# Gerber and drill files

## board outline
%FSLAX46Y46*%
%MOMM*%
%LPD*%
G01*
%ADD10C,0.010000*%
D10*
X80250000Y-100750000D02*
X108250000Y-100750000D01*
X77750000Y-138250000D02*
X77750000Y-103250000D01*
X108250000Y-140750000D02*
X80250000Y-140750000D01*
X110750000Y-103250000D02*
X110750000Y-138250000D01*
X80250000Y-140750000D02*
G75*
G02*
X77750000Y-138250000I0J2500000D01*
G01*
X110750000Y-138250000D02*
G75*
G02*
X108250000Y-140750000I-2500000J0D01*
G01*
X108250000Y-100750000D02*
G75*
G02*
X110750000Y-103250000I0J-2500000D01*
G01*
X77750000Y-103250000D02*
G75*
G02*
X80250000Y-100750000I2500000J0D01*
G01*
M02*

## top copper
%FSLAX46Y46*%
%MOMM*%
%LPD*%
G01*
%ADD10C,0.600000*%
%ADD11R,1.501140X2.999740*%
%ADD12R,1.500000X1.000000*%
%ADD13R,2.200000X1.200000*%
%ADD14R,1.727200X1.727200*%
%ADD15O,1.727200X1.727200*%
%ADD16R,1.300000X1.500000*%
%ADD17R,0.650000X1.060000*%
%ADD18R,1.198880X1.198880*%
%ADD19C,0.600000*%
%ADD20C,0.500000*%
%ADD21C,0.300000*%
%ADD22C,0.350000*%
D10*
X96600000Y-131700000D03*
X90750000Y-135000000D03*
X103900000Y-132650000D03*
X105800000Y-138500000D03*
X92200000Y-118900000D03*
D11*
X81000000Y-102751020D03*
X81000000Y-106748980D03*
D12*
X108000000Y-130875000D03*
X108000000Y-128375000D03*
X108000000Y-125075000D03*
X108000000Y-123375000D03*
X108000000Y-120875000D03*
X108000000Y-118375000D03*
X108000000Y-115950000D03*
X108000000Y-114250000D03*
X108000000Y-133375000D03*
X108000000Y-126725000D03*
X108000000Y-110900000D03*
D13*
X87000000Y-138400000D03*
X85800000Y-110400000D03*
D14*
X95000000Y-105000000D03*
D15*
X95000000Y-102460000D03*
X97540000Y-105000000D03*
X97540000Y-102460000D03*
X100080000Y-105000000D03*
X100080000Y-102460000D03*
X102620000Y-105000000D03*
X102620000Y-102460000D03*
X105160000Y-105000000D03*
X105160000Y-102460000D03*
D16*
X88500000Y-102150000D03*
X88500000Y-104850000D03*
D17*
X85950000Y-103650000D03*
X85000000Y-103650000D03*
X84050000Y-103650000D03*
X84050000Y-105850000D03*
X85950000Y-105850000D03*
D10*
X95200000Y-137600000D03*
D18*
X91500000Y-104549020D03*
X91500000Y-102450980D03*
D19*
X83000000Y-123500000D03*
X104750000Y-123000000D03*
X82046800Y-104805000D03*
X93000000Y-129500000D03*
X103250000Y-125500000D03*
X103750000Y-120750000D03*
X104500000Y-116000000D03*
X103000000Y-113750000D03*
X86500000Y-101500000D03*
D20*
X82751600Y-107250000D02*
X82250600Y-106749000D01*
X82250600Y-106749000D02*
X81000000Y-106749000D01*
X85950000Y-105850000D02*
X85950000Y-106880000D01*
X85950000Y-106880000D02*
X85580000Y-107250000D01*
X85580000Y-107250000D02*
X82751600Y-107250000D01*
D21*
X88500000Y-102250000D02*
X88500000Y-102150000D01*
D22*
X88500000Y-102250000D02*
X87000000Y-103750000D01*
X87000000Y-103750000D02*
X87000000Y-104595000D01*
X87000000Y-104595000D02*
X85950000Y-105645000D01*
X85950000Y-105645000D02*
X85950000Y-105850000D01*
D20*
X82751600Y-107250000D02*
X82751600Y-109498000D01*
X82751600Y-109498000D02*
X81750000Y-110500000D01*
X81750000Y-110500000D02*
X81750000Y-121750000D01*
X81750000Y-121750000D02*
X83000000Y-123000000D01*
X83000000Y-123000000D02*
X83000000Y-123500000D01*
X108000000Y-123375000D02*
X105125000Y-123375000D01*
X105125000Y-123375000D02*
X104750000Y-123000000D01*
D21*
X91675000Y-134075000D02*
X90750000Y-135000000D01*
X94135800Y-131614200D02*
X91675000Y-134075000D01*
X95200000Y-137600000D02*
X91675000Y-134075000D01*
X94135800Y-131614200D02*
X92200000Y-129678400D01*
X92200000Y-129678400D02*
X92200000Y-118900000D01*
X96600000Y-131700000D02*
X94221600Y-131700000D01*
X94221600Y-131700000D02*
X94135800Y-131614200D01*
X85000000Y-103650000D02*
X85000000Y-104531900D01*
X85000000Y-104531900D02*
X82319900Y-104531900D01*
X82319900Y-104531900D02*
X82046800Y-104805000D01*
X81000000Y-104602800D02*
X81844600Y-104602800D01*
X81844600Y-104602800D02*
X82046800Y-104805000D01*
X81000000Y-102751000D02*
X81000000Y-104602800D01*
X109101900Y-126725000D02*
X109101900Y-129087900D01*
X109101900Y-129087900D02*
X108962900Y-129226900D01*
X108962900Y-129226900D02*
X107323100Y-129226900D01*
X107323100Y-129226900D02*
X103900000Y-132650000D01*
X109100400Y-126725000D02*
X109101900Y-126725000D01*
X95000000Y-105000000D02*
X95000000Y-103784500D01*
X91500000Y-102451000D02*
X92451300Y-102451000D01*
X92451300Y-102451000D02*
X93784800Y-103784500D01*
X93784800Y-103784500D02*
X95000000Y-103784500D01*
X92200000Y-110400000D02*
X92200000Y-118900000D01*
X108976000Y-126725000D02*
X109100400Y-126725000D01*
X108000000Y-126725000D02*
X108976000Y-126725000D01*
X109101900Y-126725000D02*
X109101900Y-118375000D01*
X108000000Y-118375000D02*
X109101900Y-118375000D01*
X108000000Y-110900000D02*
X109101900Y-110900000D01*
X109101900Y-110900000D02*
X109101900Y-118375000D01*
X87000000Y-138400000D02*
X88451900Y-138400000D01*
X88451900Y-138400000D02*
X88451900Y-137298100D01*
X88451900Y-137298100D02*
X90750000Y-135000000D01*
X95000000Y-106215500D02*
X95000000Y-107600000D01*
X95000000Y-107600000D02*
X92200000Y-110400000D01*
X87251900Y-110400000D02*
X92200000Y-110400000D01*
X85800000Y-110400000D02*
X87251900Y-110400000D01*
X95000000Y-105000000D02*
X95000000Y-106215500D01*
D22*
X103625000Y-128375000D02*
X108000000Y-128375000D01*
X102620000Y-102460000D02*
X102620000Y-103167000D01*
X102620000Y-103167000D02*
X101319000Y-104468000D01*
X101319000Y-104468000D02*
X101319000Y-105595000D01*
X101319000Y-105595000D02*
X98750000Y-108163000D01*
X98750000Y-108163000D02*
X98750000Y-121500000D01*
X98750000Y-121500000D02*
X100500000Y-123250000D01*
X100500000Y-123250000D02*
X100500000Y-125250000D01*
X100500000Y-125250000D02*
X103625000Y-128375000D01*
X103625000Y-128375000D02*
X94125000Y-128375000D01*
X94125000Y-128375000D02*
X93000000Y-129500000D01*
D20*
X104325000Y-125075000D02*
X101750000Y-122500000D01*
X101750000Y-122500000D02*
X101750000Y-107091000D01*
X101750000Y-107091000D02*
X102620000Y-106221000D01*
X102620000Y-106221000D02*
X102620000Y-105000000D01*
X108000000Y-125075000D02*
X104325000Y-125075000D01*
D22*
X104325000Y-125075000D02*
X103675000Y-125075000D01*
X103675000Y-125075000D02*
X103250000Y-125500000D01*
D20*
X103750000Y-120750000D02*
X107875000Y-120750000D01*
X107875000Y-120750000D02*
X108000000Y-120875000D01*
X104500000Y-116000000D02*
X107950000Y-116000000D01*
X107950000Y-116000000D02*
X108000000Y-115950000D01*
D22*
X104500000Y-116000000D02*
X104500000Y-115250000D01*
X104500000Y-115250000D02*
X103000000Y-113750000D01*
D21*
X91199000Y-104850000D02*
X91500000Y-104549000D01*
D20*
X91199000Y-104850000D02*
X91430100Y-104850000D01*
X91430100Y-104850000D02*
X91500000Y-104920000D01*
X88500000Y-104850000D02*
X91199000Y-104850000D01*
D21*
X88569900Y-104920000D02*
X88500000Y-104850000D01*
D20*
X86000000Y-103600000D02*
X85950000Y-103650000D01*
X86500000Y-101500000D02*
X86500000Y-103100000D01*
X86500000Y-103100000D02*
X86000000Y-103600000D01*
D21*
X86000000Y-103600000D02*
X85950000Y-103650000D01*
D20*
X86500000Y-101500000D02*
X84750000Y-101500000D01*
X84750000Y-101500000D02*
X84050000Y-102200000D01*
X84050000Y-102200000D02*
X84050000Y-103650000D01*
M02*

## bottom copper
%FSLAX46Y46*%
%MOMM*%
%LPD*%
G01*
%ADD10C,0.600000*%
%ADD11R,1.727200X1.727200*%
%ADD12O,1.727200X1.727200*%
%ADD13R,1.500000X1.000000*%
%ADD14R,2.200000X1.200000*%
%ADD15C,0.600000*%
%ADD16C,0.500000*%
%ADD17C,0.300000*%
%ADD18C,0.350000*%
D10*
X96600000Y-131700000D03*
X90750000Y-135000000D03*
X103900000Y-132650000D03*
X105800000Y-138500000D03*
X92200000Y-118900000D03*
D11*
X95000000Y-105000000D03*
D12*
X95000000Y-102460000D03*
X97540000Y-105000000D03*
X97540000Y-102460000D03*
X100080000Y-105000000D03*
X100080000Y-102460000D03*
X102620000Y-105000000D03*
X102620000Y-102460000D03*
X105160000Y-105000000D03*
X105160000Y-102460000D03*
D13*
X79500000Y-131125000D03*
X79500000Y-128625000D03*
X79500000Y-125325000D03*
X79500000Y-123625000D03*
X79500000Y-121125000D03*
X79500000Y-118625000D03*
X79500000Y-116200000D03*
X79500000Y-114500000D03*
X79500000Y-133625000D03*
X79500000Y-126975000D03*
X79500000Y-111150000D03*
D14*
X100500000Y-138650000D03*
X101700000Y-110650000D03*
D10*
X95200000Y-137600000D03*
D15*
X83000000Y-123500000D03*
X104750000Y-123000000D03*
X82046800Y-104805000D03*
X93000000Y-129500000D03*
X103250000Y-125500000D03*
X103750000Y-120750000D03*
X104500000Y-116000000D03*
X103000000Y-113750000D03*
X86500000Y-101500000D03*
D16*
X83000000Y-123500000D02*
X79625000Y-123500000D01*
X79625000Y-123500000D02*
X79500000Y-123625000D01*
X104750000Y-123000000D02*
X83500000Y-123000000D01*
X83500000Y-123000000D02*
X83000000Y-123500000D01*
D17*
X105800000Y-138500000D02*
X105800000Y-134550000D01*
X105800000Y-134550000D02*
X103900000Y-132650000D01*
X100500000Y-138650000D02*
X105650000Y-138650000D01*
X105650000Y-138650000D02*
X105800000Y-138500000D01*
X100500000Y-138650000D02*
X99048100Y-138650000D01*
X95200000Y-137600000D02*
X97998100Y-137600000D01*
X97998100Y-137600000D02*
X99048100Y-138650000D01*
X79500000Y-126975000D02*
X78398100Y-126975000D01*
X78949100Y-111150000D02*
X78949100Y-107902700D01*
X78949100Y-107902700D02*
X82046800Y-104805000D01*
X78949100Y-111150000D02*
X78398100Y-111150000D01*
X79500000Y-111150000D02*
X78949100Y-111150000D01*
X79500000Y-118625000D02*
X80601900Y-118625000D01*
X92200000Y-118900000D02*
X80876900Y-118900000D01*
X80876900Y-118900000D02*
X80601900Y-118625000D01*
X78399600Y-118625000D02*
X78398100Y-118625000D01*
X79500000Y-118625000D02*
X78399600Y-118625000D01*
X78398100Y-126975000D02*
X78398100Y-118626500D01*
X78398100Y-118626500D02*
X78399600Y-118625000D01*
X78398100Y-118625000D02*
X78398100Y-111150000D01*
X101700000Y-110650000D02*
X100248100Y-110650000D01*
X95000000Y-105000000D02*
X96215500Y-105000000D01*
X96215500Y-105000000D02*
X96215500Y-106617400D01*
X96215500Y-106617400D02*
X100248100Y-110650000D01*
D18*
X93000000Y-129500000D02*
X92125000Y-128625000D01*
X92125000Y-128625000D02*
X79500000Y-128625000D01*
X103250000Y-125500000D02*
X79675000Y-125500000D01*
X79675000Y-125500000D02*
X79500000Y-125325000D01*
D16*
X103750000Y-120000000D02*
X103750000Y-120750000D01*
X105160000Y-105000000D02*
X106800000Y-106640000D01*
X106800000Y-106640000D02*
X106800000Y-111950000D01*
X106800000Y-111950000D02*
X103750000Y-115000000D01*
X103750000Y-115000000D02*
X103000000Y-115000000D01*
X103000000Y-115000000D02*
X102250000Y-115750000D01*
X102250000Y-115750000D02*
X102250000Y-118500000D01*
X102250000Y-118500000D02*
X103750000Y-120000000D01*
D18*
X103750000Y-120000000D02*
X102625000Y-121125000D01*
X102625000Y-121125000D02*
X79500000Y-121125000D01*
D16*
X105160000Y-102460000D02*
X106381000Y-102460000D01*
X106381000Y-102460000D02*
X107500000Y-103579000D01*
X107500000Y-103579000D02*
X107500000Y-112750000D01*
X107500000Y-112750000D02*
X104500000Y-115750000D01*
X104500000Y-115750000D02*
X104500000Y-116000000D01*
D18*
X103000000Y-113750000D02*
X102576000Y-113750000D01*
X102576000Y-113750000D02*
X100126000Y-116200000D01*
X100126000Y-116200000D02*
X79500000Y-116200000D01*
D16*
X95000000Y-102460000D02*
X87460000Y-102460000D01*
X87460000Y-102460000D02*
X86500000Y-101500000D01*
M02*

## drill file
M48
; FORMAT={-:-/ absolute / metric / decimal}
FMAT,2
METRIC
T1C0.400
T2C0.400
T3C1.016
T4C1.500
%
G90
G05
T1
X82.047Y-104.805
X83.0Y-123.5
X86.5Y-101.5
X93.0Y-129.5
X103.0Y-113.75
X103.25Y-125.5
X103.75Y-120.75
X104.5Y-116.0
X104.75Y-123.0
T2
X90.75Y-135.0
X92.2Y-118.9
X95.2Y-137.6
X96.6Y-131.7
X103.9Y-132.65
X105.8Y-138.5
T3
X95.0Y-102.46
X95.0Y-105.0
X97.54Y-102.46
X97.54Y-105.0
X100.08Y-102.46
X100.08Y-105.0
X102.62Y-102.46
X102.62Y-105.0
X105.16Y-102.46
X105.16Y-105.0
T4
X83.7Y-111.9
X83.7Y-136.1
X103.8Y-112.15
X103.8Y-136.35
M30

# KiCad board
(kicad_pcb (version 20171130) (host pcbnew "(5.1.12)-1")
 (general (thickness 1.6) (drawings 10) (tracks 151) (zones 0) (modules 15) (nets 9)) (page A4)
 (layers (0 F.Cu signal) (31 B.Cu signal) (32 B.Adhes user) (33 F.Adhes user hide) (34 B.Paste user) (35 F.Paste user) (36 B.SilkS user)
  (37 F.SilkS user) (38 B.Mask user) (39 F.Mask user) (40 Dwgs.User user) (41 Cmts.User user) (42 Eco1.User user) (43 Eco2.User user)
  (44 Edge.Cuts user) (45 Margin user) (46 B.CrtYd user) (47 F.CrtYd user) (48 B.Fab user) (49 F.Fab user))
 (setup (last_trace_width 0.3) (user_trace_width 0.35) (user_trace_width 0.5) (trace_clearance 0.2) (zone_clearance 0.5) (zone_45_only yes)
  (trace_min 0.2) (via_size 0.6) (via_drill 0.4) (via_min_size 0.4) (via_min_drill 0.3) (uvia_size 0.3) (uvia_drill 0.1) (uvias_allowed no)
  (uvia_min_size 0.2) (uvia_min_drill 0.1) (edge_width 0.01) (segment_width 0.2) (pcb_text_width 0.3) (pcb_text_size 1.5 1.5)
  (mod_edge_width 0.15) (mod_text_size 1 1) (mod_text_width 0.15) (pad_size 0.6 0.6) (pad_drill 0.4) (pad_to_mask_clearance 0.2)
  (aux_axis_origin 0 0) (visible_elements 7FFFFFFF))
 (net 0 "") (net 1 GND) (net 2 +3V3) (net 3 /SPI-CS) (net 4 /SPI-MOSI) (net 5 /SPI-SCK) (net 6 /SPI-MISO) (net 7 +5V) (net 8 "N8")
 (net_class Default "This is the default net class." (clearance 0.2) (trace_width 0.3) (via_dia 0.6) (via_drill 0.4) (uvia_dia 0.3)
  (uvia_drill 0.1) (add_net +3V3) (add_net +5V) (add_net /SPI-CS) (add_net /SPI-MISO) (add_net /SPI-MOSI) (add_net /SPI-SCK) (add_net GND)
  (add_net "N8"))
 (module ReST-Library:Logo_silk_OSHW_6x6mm (layer B.Cu) (at 86.868 123.444 270)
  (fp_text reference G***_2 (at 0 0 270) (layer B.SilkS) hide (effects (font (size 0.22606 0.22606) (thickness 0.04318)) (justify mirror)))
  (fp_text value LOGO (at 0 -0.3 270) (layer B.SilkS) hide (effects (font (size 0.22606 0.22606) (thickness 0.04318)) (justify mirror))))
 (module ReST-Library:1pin (layer F.Cu) (at 96.6 131.7) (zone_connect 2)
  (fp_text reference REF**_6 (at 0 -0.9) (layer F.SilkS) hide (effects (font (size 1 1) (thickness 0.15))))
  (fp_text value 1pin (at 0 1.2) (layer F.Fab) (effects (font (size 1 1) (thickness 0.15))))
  (pad GND thru_hole circle (at 0 0) (size 0.6 0.6) (drill 0.4) (layers *.Cu *.Mask F.SilkS) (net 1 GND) (zone_connect 2)))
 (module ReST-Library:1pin (layer F.Cu) (at 90.75 135) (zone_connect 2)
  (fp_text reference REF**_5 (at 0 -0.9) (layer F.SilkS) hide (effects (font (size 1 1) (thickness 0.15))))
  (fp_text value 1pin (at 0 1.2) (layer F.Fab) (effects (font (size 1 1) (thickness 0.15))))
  (pad GND thru_hole circle (at 0 0) (size 0.6 0.6) (drill 0.4) (layers *.Cu *.Mask F.SilkS) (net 1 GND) (zone_connect 2)))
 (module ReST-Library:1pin (layer F.Cu) (at 103.9 132.65) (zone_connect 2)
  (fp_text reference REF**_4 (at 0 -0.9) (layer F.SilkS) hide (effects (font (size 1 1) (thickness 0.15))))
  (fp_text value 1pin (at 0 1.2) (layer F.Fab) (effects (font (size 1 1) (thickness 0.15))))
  (pad GND thru_hole circle (at 0 0) (size 0.6 0.6) (drill 0.4) (layers *.Cu *.Mask F.SilkS) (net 1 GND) (zone_connect 2)))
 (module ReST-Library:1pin (layer F.Cu) (at 105.8 138.5) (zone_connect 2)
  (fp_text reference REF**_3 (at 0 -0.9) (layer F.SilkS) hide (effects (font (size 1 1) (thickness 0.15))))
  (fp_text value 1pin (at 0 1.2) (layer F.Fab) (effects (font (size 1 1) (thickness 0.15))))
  (pad GND thru_hole circle (at 0 0) (size 0.6 0.6) (drill 0.4) (layers *.Cu *.Mask F.SilkS) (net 1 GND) (zone_connect 2)))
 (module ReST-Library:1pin (layer F.Cu) (at 92.2 118.9) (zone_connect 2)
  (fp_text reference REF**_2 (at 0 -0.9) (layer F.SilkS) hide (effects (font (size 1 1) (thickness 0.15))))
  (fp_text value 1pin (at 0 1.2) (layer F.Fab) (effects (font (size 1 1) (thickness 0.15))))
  (pad GND thru_hole circle (at 0 0) (size 0.6 0.6) (drill 0.4) (layers *.Cu *.Mask F.SilkS) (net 1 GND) (zone_connect 2)))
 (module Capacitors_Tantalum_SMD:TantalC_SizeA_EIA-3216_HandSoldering (layer F.Cu) (at 81 104.75 90)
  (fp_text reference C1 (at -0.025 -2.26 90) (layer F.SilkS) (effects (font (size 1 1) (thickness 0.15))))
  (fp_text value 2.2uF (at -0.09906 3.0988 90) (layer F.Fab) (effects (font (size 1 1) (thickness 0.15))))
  (pad 2 smd rect (at 1.99898 0 90) (size 2.99974 1.50114) (layers F.Cu F.Paste F.Mask) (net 1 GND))
  (pad 1 smd rect (at -1.99898 0 90) (size 2.99974 1.50114) (layers F.Cu F.Paste F.Mask) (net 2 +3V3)))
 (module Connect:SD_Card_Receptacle (layer F.Cu) (at 108 124 270) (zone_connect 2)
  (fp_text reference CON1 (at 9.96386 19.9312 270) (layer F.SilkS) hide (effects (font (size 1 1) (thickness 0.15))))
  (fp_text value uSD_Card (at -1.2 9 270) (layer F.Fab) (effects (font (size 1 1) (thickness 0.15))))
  (pad 1 smd rect (at 6.875 0 270) (size 1 1.5) (layers F.Cu F.Paste F.Mask) (zone_connect 2))
  (pad 2 smd rect (at 4.375 0 270) (size 1 1.5) (layers F.Cu F.Paste F.Mask) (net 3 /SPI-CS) (zone_connect 2))
  (pad 3 smd rect (at 1.075 0 270) (size 1 1.5) (layers F.Cu F.Paste F.Mask) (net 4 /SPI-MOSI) (zone_connect 2))
  (pad 4 smd rect (at -0.625 0 270) (size 1 1.5) (layers F.Cu F.Paste F.Mask) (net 2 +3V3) (zone_connect 2))
  (pad 5 smd rect (at -3.125 0 270) (size 1 1.5) (layers F.Cu F.Paste F.Mask) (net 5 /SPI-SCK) (zone_connect 2))
  (pad 6 smd rect (at -5.625 0 270) (size 1 1.5) (layers F.Cu F.Paste F.Mask) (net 1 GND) (zone_connect 2))
  (pad 7 smd rect (at -8.05 0 270) (size 1 1.5) (layers F.Cu F.Paste F.Mask) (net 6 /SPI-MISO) (zone_connect 2))
  (pad 8 smd rect (at -9.75 0 270) (size 1 1.5) (layers F.Cu F.Paste F.Mask) (zone_connect 2))
  (pad 9 smd rect (at 9.375 0 270) (size 1 1.5) (layers F.Cu F.Paste F.Mask) (zone_connect 2))
  (pad 10 smd rect (at 2.725 0 270) (size 1 1.5) (layers F.Cu F.Paste F.Mask) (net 1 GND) (zone_connect 2))
  (pad 11 smd rect (at -13.1 0 270) (size 1 1.5) (layers F.Cu F.Paste F.Mask) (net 1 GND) (zone_connect 2))
  (pad 12 smd rect (at 14.4 21 270) (size 1.2 2.2) (layers F.Cu F.Paste F.Mask) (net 1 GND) (zone_connect 2))
  (pad 13 smd rect (at -13.6 22.2 270) (size 1.2 2.2) (layers F.Cu F.Paste F.Mask) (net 1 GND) (zone_connect 2))
  (pad "" np_thru_hole circle (at 12.1 24.3 270) (size 1.5 1.5) (drill 1.5) (layers *.Cu *.Mask F.SilkS) (zone_connect 2))
  (pad "" np_thru_hole circle (at -12.1 24.3 270) (size 1.5 1.5) (drill 1.5) (layers *.Cu *.Mask F.SilkS) (zone_connect 2)))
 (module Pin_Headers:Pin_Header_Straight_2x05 (layer F.Cu) (at 95 105 90)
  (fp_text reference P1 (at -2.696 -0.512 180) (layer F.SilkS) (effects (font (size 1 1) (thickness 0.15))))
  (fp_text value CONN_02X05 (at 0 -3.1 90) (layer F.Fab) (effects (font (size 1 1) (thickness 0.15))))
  (pad 1 thru_hole rect (at 0 0 90) (size 1.7272 1.7272) (drill 1.016) (layers *.Cu *.Mask F.SilkS) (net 1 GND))
  (pad 2 thru_hole oval (at 2.54 0 90) (size 1.7272 1.7272) (drill 1.016) (layers *.Cu *.Mask F.SilkS) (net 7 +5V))
  (pad 3 thru_hole oval (at 0 2.54 90) (size 1.7272 1.7272) (drill 1.016) (layers *.Cu *.Mask F.SilkS))
  (pad 4 thru_hole oval (at 2.54 2.54 90) (size 1.7272 1.7272) (drill 1.016) (layers *.Cu *.Mask F.SilkS))
  (pad 5 thru_hole oval (at 0 5.08 90) (size 1.7272 1.7272) (drill 1.016) (layers *.Cu *.Mask F.SilkS))
  (pad 6 thru_hole oval (at 2.54 5.08 90) (size 1.7272 1.7272) (drill 1.016) (layers *.Cu *.Mask F.SilkS))
  (pad 7 thru_hole oval (at 0 7.62 90) (size 1.7272 1.7272) (drill 1.016) (layers *.Cu *.Mask F.SilkS) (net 4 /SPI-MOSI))
  (pad 8 thru_hole oval (at 2.54 7.62 90) (size 1.7272 1.7272) (drill 1.016) (layers *.Cu *.Mask F.SilkS) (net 3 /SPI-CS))
  (pad 9 thru_hole oval (at 0 10.16 90) (size 1.7272 1.7272) (drill 1.016) (layers *.Cu *.Mask F.SilkS) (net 5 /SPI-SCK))
  (pad 10 thru_hole oval (at 2.54 10.16 90) (size 1.7272 1.7272) (drill 1.016) (layers *.Cu *.Mask F.SilkS) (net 6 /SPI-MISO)))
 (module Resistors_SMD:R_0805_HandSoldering (layer F.Cu) (at 88.5 103.5 270)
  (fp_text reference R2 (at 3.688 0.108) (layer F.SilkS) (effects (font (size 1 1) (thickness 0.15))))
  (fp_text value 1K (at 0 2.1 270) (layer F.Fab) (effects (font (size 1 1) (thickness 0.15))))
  (pad 1 smd rect (at -1.35 0 270) (size 1.5 1.3) (layers F.Cu F.Paste F.Mask) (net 2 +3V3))
  (pad 2 smd rect (at 1.35 0 270) (size 1.5 1.3) (layers F.Cu F.Paste F.Mask) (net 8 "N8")))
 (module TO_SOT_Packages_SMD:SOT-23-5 (layer F.Cu) (at 85 104.75 270)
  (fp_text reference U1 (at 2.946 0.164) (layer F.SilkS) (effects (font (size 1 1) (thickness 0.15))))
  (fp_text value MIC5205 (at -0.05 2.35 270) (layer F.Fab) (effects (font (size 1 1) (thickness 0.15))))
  (pad 1 smd rect (at -1.1 -0.95 270) (size 1.06 0.65) (layers F.Cu F.Paste F.Mask) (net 7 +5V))
  (pad 2 smd rect (at -1.1 0 270) (size 1.06 0.65) (layers F.Cu F.Paste F.Mask) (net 1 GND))
  (pad 3 smd rect (at -1.1 0.95 270) (size 1.06 0.65) (layers F.Cu F.Paste F.Mask) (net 7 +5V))
  (pad 4 smd rect (at 1.1 0.95 270) (size 1.06 0.65) (layers F.Cu F.Paste F.Mask))
  (pad 5 smd rect (at 1.1 -0.95 270) (size 1.06 0.65) (layers F.Cu F.Paste F.Mask) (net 2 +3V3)))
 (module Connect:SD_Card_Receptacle (layer B.Cu) (at 79.5 124.25 270) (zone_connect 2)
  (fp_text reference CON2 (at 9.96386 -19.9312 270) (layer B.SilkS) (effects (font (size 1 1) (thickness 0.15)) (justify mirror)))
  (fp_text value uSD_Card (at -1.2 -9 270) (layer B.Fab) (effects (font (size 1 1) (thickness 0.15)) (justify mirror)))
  (pad 1 smd rect (at 6.875 0 270) (size 1 1.5) (layers B.Cu B.Paste B.Mask) (zone_connect 2))
  (pad 2 smd rect (at 4.375 0 270) (size 1 1.5) (layers B.Cu B.Paste B.Mask) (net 3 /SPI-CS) (zone_connect 2))
  (pad 3 smd rect (at 1.075 0 270) (size 1 1.5) (layers B.Cu B.Paste B.Mask) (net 4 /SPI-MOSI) (zone_connect 2))
  (pad 4 smd rect (at -0.625 0 270) (size 1 1.5) (layers B.Cu B.Paste B.Mask) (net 2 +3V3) (zone_connect 2))
  (pad 5 smd rect (at -3.125 0 270) (size 1 1.5) (layers B.Cu B.Paste B.Mask) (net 5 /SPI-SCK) (zone_connect 2))
  (pad 6 smd rect (at -5.625 0 270) (size 1 1.5) (layers B.Cu B.Paste B.Mask) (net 1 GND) (zone_connect 2))
  (pad 7 smd rect (at -8.05 0 270) (size 1 1.5) (layers B.Cu B.Paste B.Mask) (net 6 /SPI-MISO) (zone_connect 2))
  (pad 8 smd rect (at -9.75 0 270) (size 1 1.5) (layers B.Cu B.Paste B.Mask) (zone_connect 2))
  (pad 9 smd rect (at 9.375 0 270) (size 1 1.5) (layers B.Cu B.Paste B.Mask) (zone_connect 2))
  (pad 10 smd rect (at 2.725 0 270) (size 1 1.5) (layers B.Cu B.Paste B.Mask) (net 1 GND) (zone_connect 2))
  (pad 11 smd rect (at -13.1 0 270) (size 1 1.5) (layers B.Cu B.Paste B.Mask) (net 1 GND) (zone_connect 2))
  (pad 12 smd rect (at 14.4 -21 270) (size 1.2 2.2) (layers B.Cu B.Paste B.Mask) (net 1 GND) (zone_connect 2))
  (pad 13 smd rect (at -13.6 -22.2 270) (size 1.2 2.2) (layers B.Cu B.Paste B.Mask) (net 1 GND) (zone_connect 2))
  (pad "" np_thru_hole circle (at 12.1 -24.3 270) (size 1.5 1.5) (drill 1.5) (layers *.Cu *.Mask B.SilkS) (zone_connect 2))
  (pad "" np_thru_hole circle (at -12.1 -24.3 270) (size 1.5 1.5) (drill 1.5) (layers *.Cu *.Mask B.SilkS) (zone_connect 2)))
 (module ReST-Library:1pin (layer F.Cu) (at 95.2 137.6) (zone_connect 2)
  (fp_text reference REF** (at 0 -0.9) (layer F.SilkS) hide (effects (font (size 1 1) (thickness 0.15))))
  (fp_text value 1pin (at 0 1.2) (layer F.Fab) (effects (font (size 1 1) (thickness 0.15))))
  (pad GND thru_hole circle (at 0 0) (size 0.6 0.6) (drill 0.4) (layers *.Cu *.Mask F.SilkS) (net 1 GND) (zone_connect 2)))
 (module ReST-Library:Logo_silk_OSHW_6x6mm (layer F.Cu) (at 86.868 123.444 90)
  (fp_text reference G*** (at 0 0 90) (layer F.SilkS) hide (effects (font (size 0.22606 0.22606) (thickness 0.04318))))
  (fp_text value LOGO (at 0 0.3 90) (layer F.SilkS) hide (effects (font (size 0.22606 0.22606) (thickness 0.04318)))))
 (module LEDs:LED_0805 (layer F.Cu) (at 91.5 103.5 270)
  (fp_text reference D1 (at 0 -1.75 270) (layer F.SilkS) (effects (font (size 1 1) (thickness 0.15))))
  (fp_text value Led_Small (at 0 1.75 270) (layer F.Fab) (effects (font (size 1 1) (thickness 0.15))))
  (pad 2 smd rect (at 1.04902 0 90) (size 1.19888 1.19888) (layers F.Cu F.Paste F.Mask) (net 8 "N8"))
  (pad 1 smd rect (at -1.04902 0 90) (size 1.19888 1.19888) (layers F.Cu F.Paste F.Mask) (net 1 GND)))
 (gr_line (start 80.25 100.75) (end 108.25 100.75) (angle 90) (layer Edge.Cuts) (width 0.01))
 (gr_line (start 77.75 138.25) (end 77.75 103.25) (angle 90) (layer Edge.Cuts) (width 0.01))
 (gr_line (start 108.25 140.75) (end 80.25 140.75) (angle 90) (layer Edge.Cuts) (width 0.01))
 (gr_line (start 110.75 103.25) (end 110.75 138.25) (angle 90) (layer Edge.Cuts) (width 0.01))
 (gr_arc (start 80.25 138.25) (end 80.25 140.75) (angle 90) (layer Edge.Cuts) (width 0.01))
 (gr_arc (start 108.25 138.25) (end 110.75 138.25) (angle 90) (layer Edge.Cuts) (width 0.01))
 (gr_arc (start 108.25 103.25) (end 108.25 100.75) (angle 90) (layer Edge.Cuts) (width 0.01))
 (gr_arc (start 80.25 103.25) (end 77.75 103.25) (angle 90) (layer Edge.Cuts) (width 0.01))
 (segment (start 82.7516 107.25) (end 82.2506 106.749) (width 0.5) (layer F.Cu) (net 2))
 (segment (start 82.2506 106.749) (end 81 106.749) (width 0.5) (layer F.Cu) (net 2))
 (segment (start 85.95 105.85) (end 85.95 106.88) (width 0.5) (layer F.Cu) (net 2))
 (segment (start 85.95 106.88) (end 85.58 107.25) (width 0.5) (layer F.Cu) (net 2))
 (segment (start 85.58 107.25) (end 82.7516 107.25) (width 0.5) (layer F.Cu) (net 2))
 (segment (start 88.5 102.25) (end 88.5 102.15) (width 0.3) (layer F.Cu) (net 2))
 (segment (start 88.5 102.25) (end 87 103.75) (width 0.35) (layer F.Cu) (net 2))
 (segment (start 87 103.75) (end 87 104.595) (width 0.35) (layer F.Cu) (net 2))
 (segment (start 87 104.595) (end 85.95 105.645) (width 0.35) (layer F.Cu) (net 2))
 (segment (start 85.95 105.645) (end 85.95 105.85) (width 0.35) (layer F.Cu) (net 2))
 (segment (start 82.7516 107.25) (end 82.7516 109.498) (width 0.5) (layer F.Cu) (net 2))
 (segment (start 82.7516 109.498) (end 81.75 110.5) (width 0.5) (layer F.Cu) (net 2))
 (segment (start 81.75 110.5) (end 81.75 121.75) (width 0.5) (layer F.Cu) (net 2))
 (segment (start 81.75 121.75) (end 83 123) (width 0.5) (layer F.Cu) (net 2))
 (segment (start 83 123) (end 83 123.5) (width 0.5) (layer F.Cu) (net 2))
 (segment (start 83 123.5) (end 79.625 123.5) (width 0.5) (layer B.Cu) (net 2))
 (segment (start 79.625 123.5) (end 79.5 123.625) (width 0.5) (layer B.Cu) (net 2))
 (segment (start 108 123.375) (end 105.125 123.375) (width 0.5) (layer F.Cu) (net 2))
 (segment (start 105.125 123.375) (end 104.75 123) (width 0.5) (layer F.Cu) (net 2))
 (segment (start 104.75 123) (end 83.5 123) (width 0.5) (layer B.Cu) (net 2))
 (segment (start 83.5 123) (end 83 123.5) (width 0.5) (layer B.Cu) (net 2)) (via (at 83 123.5) (size 0.6) (layers F.Cu B.Cu) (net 2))
 (via (at 104.75 123) (size 0.6) (layers F.Cu B.Cu) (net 2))
 (segment (start 105.8 138.5) (end 105.8 134.55) (width 0.3) (layer B.Cu) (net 1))
 (segment (start 105.8 134.55) (end 103.9 132.65) (width 0.3) (layer B.Cu) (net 1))
 (segment (start 100.5 138.65) (end 105.65 138.65) (width 0.3) (layer B.Cu) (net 1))
 (segment (start 105.65 138.65) (end 105.8 138.5) (width 0.3) (layer B.Cu) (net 1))
 (segment (start 100.5 138.65) (end 99.0481 138.65) (width 0.3) (layer B.Cu) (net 1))
 (segment (start 95.2 137.6) (end 97.9981 137.6) (width 0.3) (layer B.Cu) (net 1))
 (segment (start 97.9981 137.6) (end 99.0481 138.65) (width 0.3) (layer B.Cu) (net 1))
 (segment (start 91.675 134.075) (end 90.75 135) (width 0.3) (layer F.Cu) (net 1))
 (segment (start 94.1358 131.6142) (end 91.675 134.075) (width 0.3) (layer F.Cu) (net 1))
 (segment (start 95.2 137.6) (end 91.675 134.075) (width 0.3) (layer F.Cu) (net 1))
 (segment (start 94.1358 131.6142) (end 92.2 129.6784) (width 0.3) (layer F.Cu) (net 1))
 (segment (start 92.2 129.6784) (end 92.2 118.9) (width 0.3) (layer F.Cu) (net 1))
 (segment (start 96.6 131.7) (end 94.2216 131.7) (width 0.3) (layer F.Cu) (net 1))
 (segment (start 94.2216 131.7) (end 94.1358 131.6142) (width 0.3) (layer F.Cu) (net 1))
 (segment (start 79.5 126.975) (end 78.3981 126.975) (width 0.3) (layer B.Cu) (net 1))
 (segment (start 85 103.65) (end 85 104.5319) (width 0.3) (layer F.Cu) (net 1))
 (segment (start 85 104.5319) (end 82.3199 104.5319) (width 0.3) (layer F.Cu) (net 1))
 (segment (start 82.3199 104.5319) (end 82.0468 104.805) (width 0.3) (layer F.Cu) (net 1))
 (segment (start 81 104.6028) (end 81.8446 104.6028) (width 0.3) (layer F.Cu) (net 1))
 (segment (start 81.8446 104.6028) (end 82.0468 104.805) (width 0.3) (layer F.Cu) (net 1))
 (segment (start 78.9491 111.15) (end 78.9491 107.9027) (width 0.3) (layer B.Cu) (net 1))
 (segment (start 78.9491 107.9027) (end 82.0468 104.805) (width 0.3) (layer B.Cu) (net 1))
 (segment (start 81 102.751) (end 81 104.6028) (width 0.3) (layer F.Cu) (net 1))
 (segment (start 78.9491 111.15) (end 78.3981 111.15) (width 0.3) (layer B.Cu) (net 1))
 (segment (start 79.5 111.15) (end 78.9491 111.15) (width 0.3) (layer B.Cu) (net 1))
 (segment (start 109.1019 126.725) (end 109.1019 129.0879) (width 0.3) (layer F.Cu) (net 1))
 (segment (start 109.1019 129.0879) (end 108.9629 129.2269) (width 0.3) (layer F.Cu) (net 1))
 (segment (start 108.9629 129.2269) (end 107.3231 129.2269) (width 0.3) (layer F.Cu) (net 1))
 (segment (start 107.3231 129.2269) (end 103.9 132.65) (width 0.3) (layer F.Cu) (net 1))
 (segment (start 109.1004 126.725) (end 109.1019 126.725) (width 0.3) (layer F.Cu) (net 1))
 (segment (start 95 105) (end 95 103.7845) (width 0.3) (layer F.Cu) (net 1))
 (segment (start 91.5 102.451) (end 92.4513 102.451) (width 0.3) (layer F.Cu) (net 1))
 (segment (start 92.4513 102.451) (end 93.7848 103.7845) (width 0.3) (layer F.Cu) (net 1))
 (segment (start 93.7848 103.7845) (end 95 103.7845) (width 0.3) (layer F.Cu) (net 1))
 (segment (start 79.5 118.625) (end 80.6019 118.625) (width 0.3) (layer B.Cu) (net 1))
 (segment (start 92.2 118.9) (end 80.8769 118.9) (width 0.3) (layer B.Cu) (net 1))
 (segment (start 80.8769 118.9) (end 80.6019 118.625) (width 0.3) (layer B.Cu) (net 1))
 (segment (start 78.3996 118.625) (end 78.3981 118.625) (width 0.3) (layer B.Cu) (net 1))
 (segment (start 79.5 118.625) (end 78.3996 118.625) (width 0.3) (layer B.Cu) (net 1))
 (segment (start 78.3981 126.975) (end 78.3981 118.6265) (width 0.3) (layer B.Cu) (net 1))
 (segment (start 78.3981 118.6265) (end 78.3996 118.625) (width 0.3) (layer B.Cu) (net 1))
 (segment (start 78.3981 118.625) (end 78.3981 111.15) (width 0.3) (layer B.Cu) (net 1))
 (segment (start 92.2 110.4) (end 92.2 118.9) (width 0.3) (layer F.Cu) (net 1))
 (segment (start 108.976 126.725) (end 109.1004 126.725) (width 0.3) (layer F.Cu) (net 1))
 (segment (start 108 126.725) (end 108.976 126.725) (width 0.3) (layer F.Cu) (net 1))
 (segment (start 109.1019 126.725) (end 109.1019 118.375) (width 0.3) (layer F.Cu) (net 1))
 (segment (start 108 118.375) (end 109.1019 118.375) (width 0.3) (layer F.Cu) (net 1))
 (segment (start 108 110.9) (end 109.1019 110.9) (width 0.3) (layer F.Cu) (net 1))
 (segment (start 109.1019 110.9) (end 109.1019 118.375) (width 0.3) (layer F.Cu) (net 1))
 (segment (start 87 138.4) (end 88.4519 138.4) (width 0.3) (layer F.Cu) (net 1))
 (segment (start 88.4519 138.4) (end 88.4519 137.2981) (width 0.3) (layer F.Cu) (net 1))
 (segment (start 88.4519 137.2981) (end 90.75 135) (width 0.3) (layer F.Cu) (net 1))
 (segment (start 95 106.2155) (end 95 107.6) (width 0.3) (layer F.Cu) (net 1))
 (segment (start 95 107.6) (end 92.2 110.4) (width 0.3) (layer F.Cu) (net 1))
 (segment (start 87.2519 110.4) (end 92.2 110.4) (width 0.3) (layer F.Cu) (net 1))
 (segment (start 85.8 110.4) (end 87.2519 110.4) (width 0.3) (layer F.Cu) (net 1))
 (segment (start 95 105) (end 95 106.2155) (width 0.3) (layer F.Cu) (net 1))
 (segment (start 101.7 110.65) (end 100.2481 110.65) (width 0.3) (layer B.Cu) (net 1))
 (segment (start 95 105) (end 96.2155 105) (width 0.3) (layer B.Cu) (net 1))
 (segment (start 96.2155 105) (end 96.2155 106.6174) (width 0.3) (layer B.Cu) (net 1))
 (segment (start 96.2155 106.6174) (end 100.2481 110.65) (width 0.3) (layer B.Cu) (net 1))
 (via (at 82.0468 104.805) (size 0.6) (layers F.Cu B.Cu) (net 1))
 (segment (start 103.625 128.375) (end 108 128.375) (width 0.35) (layer F.Cu) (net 3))
 (segment (start 102.62 102.46) (end 102.62 103.167) (width 0.35) (layer F.Cu) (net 3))
 (segment (start 102.62 103.167) (end 101.319 104.468) (width 0.35) (layer F.Cu) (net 3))
 (segment (start 101.319 104.468) (end 101.319 105.595) (width 0.35) (layer F.Cu) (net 3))
 (segment (start 101.319 105.595) (end 98.75 108.163) (width 0.35) (layer F.Cu) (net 3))
 (segment (start 98.75 108.163) (end 98.75 121.5) (width 0.35) (layer F.Cu) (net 3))
 (segment (start 98.75 121.5) (end 100.5 123.25) (width 0.35) (layer F.Cu) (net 3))
 (segment (start 100.5 123.25) (end 100.5 125.25) (width 0.35) (layer F.Cu) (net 3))
 (segment (start 100.5 125.25) (end 103.625 128.375) (width 0.35) (layer F.Cu) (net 3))
 (segment (start 103.625 128.375) (end 94.125 128.375) (width 0.35) (layer F.Cu) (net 3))
 (segment (start 94.125 128.375) (end 93 129.5) (width 0.35) (layer F.Cu) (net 3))
 (segment (start 93 129.5) (end 92.125 128.625) (width 0.35) (layer B.Cu) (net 3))
 (segment (start 92.125 128.625) (end 79.5 128.625) (width 0.35) (layer B.Cu) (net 3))
 (via (at 93 129.5) (size 0.6) (layers F.Cu B.Cu) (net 3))
 (segment (start 104.325 125.075) (end 101.75 122.5) (width 0.5) (layer F.Cu) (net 4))
 (segment (start 101.75 122.5) (end 101.75 107.091) (width 0.5) (layer F.Cu) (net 4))
 (segment (start 101.75 107.091) (end 102.62 106.221) (width 0.5) (layer F.Cu) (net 4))
 (segment (start 102.62 106.221) (end 102.62 105) (width 0.5) (layer F.Cu) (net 4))
 (segment (start 108 125.075) (end 104.325 125.075) (width 0.5) (layer F.Cu) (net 4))
 (segment (start 104.325 125.075) (end 103.675 125.075) (width 0.35) (layer F.Cu) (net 4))
 (segment (start 103.675 125.075) (end 103.25 125.5) (width 0.35) (layer F.Cu) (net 4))
 (segment (start 103.25 125.5) (end 79.675 125.5) (width 0.35) (layer B.Cu) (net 4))
 (segment (start 79.675 125.5) (end 79.5 125.325) (width 0.35) (layer B.Cu) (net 4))
 (via (at 103.25 125.5) (size 0.6) (layers F.Cu B.Cu) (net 4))
 (segment (start 103.75 120) (end 103.75 120.75) (width 0.5) (layer B.Cu) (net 5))
 (segment (start 105.16 105) (end 106.8 106.64) (width 0.5) (layer B.Cu) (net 5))
 (segment (start 106.8 106.64) (end 106.8 111.95) (width 0.5) (layer B.Cu) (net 5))
 (segment (start 106.8 111.95) (end 103.75 115) (width 0.5) (layer B.Cu) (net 5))
 (segment (start 103.75 115) (end 103 115) (width 0.5) (layer B.Cu) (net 5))
 (segment (start 103 115) (end 102.25 115.75) (width 0.5) (layer B.Cu) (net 5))
 (segment (start 102.25 115.75) (end 102.25 118.5) (width 0.5) (layer B.Cu) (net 5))
 (segment (start 102.25 118.5) (end 103.75 120) (width 0.5) (layer B.Cu) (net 5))
 (segment (start 103.75 120.75) (end 107.875 120.75) (width 0.5) (layer F.Cu) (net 5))
 (segment (start 107.875 120.75) (end 108 120.875) (width 0.5) (layer F.Cu) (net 5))
 (segment (start 103.75 120) (end 102.625 121.125) (width 0.35) (layer B.Cu) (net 5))
 (segment (start 102.625 121.125) (end 79.5 121.125) (width 0.35) (layer B.Cu) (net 5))
 (via (at 103.75 120.75) (size 0.6) (layers F.Cu B.Cu) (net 5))
 (segment (start 105.16 102.46) (end 106.381 102.46) (width 0.5) (layer B.Cu) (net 6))
 (segment (start 106.381 102.46) (end 107.5 103.579) (width 0.5) (layer B.Cu) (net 6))
 (segment (start 107.5 103.579) (end 107.5 112.75) (width 0.5) (layer B.Cu) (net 6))
 (segment (start 107.5 112.75) (end 104.5 115.75) (width 0.5) (layer B.Cu) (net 6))
 (segment (start 104.5 115.75) (end 104.5 116) (width 0.5) (layer B.Cu) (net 6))
 (segment (start 104.5 116) (end 107.95 116) (width 0.5) (layer F.Cu) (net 6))
 (segment (start 107.95 116) (end 108 115.95) (width 0.5) (layer F.Cu) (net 6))
 (segment (start 104.5 116) (end 104.5 115.25) (width 0.35) (layer F.Cu) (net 6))
 (segment (start 104.5 115.25) (end 103 113.75) (width 0.35) (layer F.Cu) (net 6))
 (segment (start 103 113.75) (end 102.576 113.75) (width 0.35) (layer B.Cu) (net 6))
 (segment (start 102.576 113.75) (end 100.126 116.2) (width 0.35) (layer B.Cu) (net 6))
 (segment (start 100.126 116.2) (end 79.5 116.2) (width 0.35) (layer B.Cu) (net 6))
 (via (at 104.5 116) (size 0.6) (layers F.Cu B.Cu) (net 6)) (via (at 103 113.75) (size 0.6) (layers F.Cu B.Cu) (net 6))
 (segment (start 91.199 104.85) (end 91.5 104.549) (width 0.3) (layer F.Cu) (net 8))
 (segment (start 91.199 104.85) (end 91.4301 104.85) (width 0.5) (layer F.Cu) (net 8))
 (segment (start 91.4301 104.85) (end 91.5 104.92) (width 0.5) (layer F.Cu) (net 8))
 (segment (start 88.5 104.85) (end 91.199 104.85) (width 0.5) (layer F.Cu) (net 8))
 (segment (start 88.5699 104.92) (end 88.5 104.85) (width 0.3) (layer F.Cu) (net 8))
 (segment (start 86 103.6) (end 85.95 103.65) (width 0.5) (layer F.Cu) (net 7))
 (segment (start 86.5 101.5) (end 86.5 103.1) (width 0.5) (layer F.Cu) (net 7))
 (segment (start 86.5 103.1) (end 86 103.6) (width 0.5) (layer F.Cu) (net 7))
 (segment (start 86 103.6) (end 85.95 103.65) (width 0.3) (layer F.Cu) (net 7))
 (segment (start 95 102.46) (end 87.46 102.46) (width 0.5) (layer B.Cu) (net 7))
 (segment (start 87.46 102.46) (end 86.5 101.5) (width 0.5) (layer B.Cu) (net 7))
 (segment (start 86.5 101.5) (end 84.75 101.5) (width 0.5) (layer F.Cu) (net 7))
 (segment (start 84.75 101.5) (end 84.05 102.2) (width 0.5) (layer F.Cu) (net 7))
 (segment (start 84.05 102.2) (end 84.05 103.65) (width 0.5) (layer F.Cu) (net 7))
 (via (at 86.5 101.5) (size 0.6) (layers F.Cu B.Cu) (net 7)))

